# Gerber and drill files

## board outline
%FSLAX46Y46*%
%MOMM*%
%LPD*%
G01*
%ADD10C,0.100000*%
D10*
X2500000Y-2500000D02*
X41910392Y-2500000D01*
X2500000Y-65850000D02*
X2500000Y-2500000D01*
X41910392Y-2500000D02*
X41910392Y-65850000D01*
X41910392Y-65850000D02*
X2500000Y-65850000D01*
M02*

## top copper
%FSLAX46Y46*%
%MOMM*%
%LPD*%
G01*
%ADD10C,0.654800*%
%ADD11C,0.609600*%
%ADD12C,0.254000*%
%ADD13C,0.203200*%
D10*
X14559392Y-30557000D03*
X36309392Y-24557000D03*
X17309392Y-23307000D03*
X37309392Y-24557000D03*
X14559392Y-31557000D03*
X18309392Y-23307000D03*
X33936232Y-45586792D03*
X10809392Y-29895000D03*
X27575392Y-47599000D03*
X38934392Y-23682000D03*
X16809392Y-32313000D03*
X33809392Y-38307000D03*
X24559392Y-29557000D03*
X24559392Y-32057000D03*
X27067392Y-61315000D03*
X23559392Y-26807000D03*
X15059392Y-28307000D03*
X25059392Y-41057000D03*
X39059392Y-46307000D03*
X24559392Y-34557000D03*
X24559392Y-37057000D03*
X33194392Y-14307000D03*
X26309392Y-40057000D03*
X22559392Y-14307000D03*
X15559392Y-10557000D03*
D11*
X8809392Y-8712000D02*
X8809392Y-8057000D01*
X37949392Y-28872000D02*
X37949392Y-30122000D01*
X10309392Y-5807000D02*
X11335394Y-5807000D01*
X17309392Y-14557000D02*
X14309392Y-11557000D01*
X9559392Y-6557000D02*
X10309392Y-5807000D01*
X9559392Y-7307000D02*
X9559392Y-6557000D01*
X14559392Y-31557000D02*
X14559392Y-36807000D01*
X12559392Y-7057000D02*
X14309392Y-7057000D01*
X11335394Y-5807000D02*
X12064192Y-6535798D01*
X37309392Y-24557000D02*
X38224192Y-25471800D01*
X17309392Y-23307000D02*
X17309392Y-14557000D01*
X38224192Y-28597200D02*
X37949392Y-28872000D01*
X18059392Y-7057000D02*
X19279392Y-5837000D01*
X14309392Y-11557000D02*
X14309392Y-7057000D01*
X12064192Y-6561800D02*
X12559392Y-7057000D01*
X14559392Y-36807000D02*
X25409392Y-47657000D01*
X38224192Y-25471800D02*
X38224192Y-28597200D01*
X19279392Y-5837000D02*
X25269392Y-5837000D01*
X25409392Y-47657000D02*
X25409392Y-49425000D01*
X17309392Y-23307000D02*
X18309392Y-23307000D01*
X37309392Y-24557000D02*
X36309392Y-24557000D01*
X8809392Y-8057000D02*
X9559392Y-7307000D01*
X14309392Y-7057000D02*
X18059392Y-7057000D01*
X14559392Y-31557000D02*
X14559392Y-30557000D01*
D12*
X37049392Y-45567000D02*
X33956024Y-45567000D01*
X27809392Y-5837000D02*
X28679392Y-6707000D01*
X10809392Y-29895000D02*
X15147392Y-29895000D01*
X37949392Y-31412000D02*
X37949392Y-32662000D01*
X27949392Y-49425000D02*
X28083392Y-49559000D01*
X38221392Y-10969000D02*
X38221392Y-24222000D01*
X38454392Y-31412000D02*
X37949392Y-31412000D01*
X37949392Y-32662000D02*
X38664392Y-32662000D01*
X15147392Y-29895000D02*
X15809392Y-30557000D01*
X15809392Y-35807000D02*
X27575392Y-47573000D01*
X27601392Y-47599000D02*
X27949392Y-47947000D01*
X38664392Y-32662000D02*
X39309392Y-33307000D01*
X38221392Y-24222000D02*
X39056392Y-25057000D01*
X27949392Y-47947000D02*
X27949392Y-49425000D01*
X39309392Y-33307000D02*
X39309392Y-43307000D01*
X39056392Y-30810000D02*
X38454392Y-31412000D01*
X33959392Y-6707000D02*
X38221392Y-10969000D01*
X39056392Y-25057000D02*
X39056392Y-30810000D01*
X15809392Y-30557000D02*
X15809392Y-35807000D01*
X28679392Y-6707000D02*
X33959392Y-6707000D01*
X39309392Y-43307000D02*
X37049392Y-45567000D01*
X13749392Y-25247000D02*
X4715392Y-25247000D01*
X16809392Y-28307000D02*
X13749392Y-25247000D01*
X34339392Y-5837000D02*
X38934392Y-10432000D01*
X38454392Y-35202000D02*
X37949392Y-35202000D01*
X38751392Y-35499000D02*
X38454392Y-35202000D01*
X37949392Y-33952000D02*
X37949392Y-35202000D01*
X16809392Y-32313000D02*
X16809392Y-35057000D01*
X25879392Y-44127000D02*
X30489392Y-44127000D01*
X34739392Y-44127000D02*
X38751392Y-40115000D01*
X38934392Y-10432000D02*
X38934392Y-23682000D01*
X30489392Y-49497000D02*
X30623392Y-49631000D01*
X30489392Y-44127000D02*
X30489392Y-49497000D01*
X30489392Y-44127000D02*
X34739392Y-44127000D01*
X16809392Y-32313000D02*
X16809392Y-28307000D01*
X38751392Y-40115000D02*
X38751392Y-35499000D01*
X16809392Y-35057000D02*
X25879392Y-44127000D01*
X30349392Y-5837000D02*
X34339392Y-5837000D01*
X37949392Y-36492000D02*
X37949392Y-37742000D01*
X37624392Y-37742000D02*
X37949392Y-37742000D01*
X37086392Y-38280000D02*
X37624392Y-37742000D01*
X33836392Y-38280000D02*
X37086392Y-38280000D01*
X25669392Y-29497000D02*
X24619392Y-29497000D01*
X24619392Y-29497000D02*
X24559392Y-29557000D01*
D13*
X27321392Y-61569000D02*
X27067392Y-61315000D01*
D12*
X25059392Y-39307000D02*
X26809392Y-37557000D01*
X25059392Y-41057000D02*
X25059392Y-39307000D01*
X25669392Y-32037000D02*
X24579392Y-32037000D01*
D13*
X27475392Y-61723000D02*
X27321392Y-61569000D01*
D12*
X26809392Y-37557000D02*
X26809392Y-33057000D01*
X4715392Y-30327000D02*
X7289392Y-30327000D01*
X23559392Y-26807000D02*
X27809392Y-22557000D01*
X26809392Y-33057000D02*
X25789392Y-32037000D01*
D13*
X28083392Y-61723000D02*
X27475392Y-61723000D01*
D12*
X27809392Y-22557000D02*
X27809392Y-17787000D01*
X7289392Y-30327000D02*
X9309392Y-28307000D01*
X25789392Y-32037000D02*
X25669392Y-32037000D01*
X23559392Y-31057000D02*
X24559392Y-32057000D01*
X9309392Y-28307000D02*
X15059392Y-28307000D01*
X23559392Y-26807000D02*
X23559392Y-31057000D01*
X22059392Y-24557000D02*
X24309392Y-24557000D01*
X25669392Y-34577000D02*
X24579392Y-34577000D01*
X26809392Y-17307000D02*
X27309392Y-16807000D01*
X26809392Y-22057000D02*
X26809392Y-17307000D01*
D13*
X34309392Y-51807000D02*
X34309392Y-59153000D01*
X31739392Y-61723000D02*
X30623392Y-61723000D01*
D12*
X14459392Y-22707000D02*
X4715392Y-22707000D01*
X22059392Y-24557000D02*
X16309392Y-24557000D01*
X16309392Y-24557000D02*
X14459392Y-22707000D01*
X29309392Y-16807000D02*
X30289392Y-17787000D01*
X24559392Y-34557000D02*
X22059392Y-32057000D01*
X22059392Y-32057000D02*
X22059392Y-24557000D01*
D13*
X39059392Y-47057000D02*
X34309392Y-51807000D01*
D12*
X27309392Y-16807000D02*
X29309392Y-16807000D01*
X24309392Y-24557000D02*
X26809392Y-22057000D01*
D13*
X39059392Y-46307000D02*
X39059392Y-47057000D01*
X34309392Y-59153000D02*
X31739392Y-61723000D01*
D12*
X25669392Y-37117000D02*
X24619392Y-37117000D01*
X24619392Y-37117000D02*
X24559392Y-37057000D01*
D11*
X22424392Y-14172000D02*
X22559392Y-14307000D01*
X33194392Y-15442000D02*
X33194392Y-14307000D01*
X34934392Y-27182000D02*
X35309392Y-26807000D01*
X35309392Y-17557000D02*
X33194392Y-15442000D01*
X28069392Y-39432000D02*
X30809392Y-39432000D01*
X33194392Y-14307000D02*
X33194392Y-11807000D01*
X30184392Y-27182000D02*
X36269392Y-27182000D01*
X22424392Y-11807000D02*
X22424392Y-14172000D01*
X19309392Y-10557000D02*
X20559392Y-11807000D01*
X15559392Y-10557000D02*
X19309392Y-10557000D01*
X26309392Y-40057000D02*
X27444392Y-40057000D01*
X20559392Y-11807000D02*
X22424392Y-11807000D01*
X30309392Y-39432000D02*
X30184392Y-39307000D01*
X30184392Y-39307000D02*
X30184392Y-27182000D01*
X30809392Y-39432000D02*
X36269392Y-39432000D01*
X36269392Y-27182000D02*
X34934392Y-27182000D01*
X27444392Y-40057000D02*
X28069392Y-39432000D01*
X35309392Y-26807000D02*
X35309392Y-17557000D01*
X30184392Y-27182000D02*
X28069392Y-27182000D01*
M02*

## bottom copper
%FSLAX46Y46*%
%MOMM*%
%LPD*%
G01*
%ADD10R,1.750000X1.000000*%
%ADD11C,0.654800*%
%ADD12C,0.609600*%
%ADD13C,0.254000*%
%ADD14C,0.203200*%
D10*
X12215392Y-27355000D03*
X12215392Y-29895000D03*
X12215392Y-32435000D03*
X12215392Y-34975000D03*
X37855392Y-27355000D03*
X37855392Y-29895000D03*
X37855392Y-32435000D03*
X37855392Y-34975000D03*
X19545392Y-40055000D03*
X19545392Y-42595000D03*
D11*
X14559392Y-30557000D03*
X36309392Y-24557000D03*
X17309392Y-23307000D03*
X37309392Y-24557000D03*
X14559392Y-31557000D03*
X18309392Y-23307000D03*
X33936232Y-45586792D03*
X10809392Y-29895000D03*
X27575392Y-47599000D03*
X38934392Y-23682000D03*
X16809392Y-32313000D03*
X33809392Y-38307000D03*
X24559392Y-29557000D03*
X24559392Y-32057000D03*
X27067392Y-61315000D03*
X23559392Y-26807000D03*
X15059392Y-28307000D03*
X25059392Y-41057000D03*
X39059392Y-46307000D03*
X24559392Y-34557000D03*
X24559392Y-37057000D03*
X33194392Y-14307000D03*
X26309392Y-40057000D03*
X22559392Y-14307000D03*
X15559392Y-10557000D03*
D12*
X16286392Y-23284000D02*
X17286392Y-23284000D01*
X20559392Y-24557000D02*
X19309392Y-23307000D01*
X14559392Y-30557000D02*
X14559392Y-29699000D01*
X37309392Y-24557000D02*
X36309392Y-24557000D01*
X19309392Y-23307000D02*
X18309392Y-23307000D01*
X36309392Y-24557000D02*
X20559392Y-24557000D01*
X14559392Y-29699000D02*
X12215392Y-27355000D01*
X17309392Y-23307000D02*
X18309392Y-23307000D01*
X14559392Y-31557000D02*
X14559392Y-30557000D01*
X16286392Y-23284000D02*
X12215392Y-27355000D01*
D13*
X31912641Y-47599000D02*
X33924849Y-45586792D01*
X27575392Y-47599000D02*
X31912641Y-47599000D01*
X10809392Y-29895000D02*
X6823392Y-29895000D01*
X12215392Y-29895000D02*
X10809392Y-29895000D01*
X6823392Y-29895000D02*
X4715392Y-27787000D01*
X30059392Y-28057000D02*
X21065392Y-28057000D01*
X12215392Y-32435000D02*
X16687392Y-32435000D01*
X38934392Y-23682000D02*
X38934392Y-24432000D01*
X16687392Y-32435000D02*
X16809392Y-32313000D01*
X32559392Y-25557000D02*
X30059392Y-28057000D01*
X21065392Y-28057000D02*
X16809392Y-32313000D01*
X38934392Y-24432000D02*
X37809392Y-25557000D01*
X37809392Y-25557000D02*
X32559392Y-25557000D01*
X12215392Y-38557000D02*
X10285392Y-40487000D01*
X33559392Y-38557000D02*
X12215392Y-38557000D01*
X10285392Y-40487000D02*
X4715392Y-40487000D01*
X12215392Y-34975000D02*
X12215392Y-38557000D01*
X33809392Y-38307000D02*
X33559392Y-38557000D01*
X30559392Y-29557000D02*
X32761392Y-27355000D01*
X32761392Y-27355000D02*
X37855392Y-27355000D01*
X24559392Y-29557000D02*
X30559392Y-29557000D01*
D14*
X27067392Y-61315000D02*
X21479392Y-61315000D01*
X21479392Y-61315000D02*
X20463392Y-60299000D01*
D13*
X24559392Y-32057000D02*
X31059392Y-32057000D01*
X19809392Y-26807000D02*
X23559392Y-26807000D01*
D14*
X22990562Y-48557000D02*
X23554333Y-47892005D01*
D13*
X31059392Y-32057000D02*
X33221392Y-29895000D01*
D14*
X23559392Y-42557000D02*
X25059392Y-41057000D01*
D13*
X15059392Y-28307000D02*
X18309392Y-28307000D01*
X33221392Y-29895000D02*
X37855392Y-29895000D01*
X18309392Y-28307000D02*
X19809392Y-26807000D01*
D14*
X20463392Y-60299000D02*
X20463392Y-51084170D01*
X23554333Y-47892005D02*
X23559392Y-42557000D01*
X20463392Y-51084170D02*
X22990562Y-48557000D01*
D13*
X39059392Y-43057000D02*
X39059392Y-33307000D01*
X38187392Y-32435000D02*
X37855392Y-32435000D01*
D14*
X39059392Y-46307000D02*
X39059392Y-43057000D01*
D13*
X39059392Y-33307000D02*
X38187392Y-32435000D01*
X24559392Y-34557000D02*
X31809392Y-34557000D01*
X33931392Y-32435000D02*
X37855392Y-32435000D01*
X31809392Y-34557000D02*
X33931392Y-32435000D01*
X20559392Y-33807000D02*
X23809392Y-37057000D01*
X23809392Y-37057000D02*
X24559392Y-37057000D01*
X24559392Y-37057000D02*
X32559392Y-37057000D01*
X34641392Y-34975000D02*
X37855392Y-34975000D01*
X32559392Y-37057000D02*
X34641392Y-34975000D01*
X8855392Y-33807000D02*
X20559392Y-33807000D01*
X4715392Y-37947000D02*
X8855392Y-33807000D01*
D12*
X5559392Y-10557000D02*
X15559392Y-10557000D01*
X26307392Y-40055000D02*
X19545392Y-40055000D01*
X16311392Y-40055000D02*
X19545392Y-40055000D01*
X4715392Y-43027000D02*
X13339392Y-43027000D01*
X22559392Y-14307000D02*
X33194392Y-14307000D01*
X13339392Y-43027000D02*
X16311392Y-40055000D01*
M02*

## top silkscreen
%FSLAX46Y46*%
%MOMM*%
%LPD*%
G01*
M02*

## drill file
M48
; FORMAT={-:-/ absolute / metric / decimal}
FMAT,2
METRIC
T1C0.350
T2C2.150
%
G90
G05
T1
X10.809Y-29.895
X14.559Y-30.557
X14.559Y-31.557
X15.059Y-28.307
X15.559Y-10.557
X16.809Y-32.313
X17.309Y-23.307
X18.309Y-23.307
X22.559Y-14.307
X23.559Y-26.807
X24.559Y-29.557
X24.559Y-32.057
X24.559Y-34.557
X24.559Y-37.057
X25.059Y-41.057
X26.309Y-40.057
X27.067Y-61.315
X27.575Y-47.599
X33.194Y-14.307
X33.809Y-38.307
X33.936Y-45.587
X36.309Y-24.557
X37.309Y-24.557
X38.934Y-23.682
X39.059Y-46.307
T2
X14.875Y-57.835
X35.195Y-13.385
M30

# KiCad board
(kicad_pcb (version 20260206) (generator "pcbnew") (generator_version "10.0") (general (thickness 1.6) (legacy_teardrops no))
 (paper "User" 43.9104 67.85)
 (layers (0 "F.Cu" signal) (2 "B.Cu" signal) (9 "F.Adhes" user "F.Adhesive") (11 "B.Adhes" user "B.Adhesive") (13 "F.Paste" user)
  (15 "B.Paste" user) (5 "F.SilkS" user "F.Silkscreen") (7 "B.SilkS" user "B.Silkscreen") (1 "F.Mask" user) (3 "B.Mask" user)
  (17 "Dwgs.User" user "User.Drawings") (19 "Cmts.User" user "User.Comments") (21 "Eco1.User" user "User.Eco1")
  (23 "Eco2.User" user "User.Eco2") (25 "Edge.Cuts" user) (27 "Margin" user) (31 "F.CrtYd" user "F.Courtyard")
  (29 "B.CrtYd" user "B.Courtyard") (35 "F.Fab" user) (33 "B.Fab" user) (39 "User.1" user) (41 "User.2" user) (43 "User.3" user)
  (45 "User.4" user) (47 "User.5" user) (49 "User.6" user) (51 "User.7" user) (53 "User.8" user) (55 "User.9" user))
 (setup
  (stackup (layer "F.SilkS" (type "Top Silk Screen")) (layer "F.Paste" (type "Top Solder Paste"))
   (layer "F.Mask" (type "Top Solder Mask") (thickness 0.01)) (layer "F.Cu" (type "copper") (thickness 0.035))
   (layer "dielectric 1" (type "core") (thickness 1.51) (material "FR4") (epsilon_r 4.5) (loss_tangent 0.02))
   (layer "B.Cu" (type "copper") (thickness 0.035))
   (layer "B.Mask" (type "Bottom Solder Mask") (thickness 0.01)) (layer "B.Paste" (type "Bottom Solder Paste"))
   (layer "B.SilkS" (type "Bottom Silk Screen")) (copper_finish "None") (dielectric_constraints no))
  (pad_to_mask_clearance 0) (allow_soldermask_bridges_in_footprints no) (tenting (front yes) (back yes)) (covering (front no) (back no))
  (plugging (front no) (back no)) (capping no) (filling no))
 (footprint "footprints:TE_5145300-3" (layer "B.Cu") (at 23.085392 34.175 -90)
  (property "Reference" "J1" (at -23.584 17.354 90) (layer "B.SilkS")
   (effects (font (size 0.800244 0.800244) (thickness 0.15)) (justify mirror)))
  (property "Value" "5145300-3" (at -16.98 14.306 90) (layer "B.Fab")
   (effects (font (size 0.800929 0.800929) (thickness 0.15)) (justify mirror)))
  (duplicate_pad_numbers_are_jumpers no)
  (pad "" np_thru_hole circle (at -20.79 -12.11 270) (size 2.15 2.15) (drill 2.15) (layers "*.Cu" "*.Mask"))
  (pad "" np_thru_hole circle (at 23.66 8.21 270) (size 2.15 2.15) (drill 2.15) (layers "*.Cu" "*.Mask"))
  (pad "C1" smd rect (at -6.82 10.87 180) (size 1.75 1) (layers "B.Cu" "B.Mask" "B.Paste") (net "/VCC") (solder_mask_margin 0.102))
  (pad "C2" smd rect (at -4.28 10.87 180) (size 1.75 1) (layers "B.Cu" "B.Mask" "B.Paste") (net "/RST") (solder_mask_margin 0.102))
  (pad "C3" smd rect (at -1.74 10.87 180) (size 1.75 1) (layers "B.Cu" "B.Mask" "B.Paste") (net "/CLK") (solder_mask_margin 0.102))
  (pad "C4" smd rect (at 0.8 10.87 180) (size 1.75 1) (layers "B.Cu" "B.Mask" "B.Paste") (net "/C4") (solder_mask_margin 0.102))
  (pad "C5" smd rect (at -6.82 -14.77 180) (size 1.75 1) (layers "B.Cu" "B.Mask" "B.Paste") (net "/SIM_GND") (solder_mask_margin 0.102))
  (pad "C6" smd rect (at -4.28 -14.77 180) (size 1.75 1) (layers "B.Cu" "B.Mask" "B.Paste") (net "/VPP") (solder_mask_margin 0.102))
  (pad "C7" smd rect (at -1.74 -14.77 180) (size 1.75 1) (layers "B.Cu" "B.Mask" "B.Paste") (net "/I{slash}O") (solder_mask_margin 0.102))
  (pad "C8" smd rect (at 0.8 -14.77 180) (size 1.75 1) (layers "B.Cu" "B.Mask" "B.Paste") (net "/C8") (solder_mask_margin 0.102))
  (pad "SW1" smd rect (at 5.88 3.54 180) (size 1.75 1) (layers "B.Cu" "B.Mask" "B.Paste") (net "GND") (solder_mask_margin 0.102))
  (pad "SW2" smd rect (at 8.42 3.54 180) (size 1.75 1) (layers "B.Cu" "B.Mask" "B.Paste") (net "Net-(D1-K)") (solder_mask_margin 0.102)))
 (gr_line (start 2.5 2.5) (end 41.910392 2.5) (stroke (width 0.1) (type default)) (layer "Edge.Cuts"))
 (gr_line (start 2.5 65.85) (end 2.5 2.5) (stroke (width 0.1) (type default)) (layer "Edge.Cuts"))
 (gr_line (start 41.910392 2.5) (end 41.910392 65.85) (stroke (width 0.1) (type default)) (layer "Edge.Cuts"))
 (gr_line (start 41.910392 65.85) (end 2.5 65.85) (stroke (width 0.1) (type default)) (layer "Edge.Cuts"))
 (segment (start 8.809392 8.712) (end 8.809392 8.057) (width 0.6096) (layer "F.Cu") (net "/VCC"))
 (segment (start 37.949392 28.872) (end 37.949392 30.122) (width 0.6096) (layer "F.Cu") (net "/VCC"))
 (segment (start 10.309392 5.807) (end 11.335394 5.807) (width 0.6096) (layer "F.Cu") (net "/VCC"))
 (segment (start 17.309392 14.557) (end 14.309392 11.557) (width 0.6096) (layer "F.Cu") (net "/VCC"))
 (segment (start 9.559392 6.557) (end 10.309392 5.807) (width 0.6096) (layer "F.Cu") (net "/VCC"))
 (segment (start 9.559392 7.307) (end 9.559392 6.557) (width 0.6096) (layer "F.Cu") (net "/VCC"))
 (segment (start 14.559392 31.557) (end 14.559392 36.807) (width 0.6096) (layer "F.Cu") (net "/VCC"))
 (segment (start 12.559392 7.057) (end 14.309392 7.057) (width 0.6096) (layer "F.Cu") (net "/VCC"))
 (segment (start 11.335394 5.807) (end 12.064192 6.535798) (width 0.6096) (layer "F.Cu") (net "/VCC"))
 (segment (start 37.309392 24.557) (end 38.224192 25.4718) (width 0.6096) (layer "F.Cu") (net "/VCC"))
 (segment (start 17.309392 23.307) (end 17.309392 14.557) (width 0.6096) (layer "F.Cu") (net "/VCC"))
 (segment (start 38.224192 28.5972) (end 37.949392 28.872) (width 0.6096) (layer "F.Cu") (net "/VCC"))
 (segment (start 18.059392 7.057) (end 19.279392 5.837) (width 0.6096) (layer "F.Cu") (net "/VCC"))
 (segment (start 14.309392 11.557) (end 14.309392 7.057) (width 0.6096) (layer "F.Cu") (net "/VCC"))
 (segment (start 12.064192 6.5618) (end 12.559392 7.057) (width 0.6096) (layer "F.Cu") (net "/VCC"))
 (segment (start 14.559392 36.807) (end 25.409392 47.657) (width 0.6096) (layer "F.Cu") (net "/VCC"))
 (segment (start 38.224192 25.4718) (end 38.224192 28.5972) (width 0.6096) (layer "F.Cu") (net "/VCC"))
 (segment (start 19.279392 5.837) (end 25.269392 5.837) (width 0.6096) (layer "F.Cu") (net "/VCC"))
 (segment (start 25.409392 47.657) (end 25.409392 49.425) (width 0.6096) (layer "F.Cu") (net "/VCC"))
 (segment (start 17.309392 23.307) (end 18.309392 23.307) (width 0.6096) (layer "F.Cu") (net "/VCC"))
 (segment (start 37.309392 24.557) (end 36.309392 24.557) (width 0.6096) (layer "F.Cu") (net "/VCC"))
 (segment (start 8.809392 8.057) (end 9.559392 7.307) (width 0.6096) (layer "F.Cu") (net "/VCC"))
 (segment (start 14.309392 7.057) (end 18.059392 7.057) (width 0.6096) (layer "F.Cu") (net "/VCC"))
 (segment (start 14.559392 31.557) (end 14.559392 30.557) (width 0.6096) (layer "F.Cu") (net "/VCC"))
 (via (at 14.559392 30.557) (size 0.6548) (drill 0.35) (layers "F.Cu" "B.Cu") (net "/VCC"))
 (via (at 36.309392 24.557) (size 0.6548) (drill 0.35) (layers "F.Cu" "B.Cu") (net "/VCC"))
 (via (at 17.309392 23.307) (size 0.6548) (drill 0.35) (layers "F.Cu" "B.Cu") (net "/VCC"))
 (via (at 37.309392 24.557) (size 0.6548) (drill 0.35) (layers "F.Cu" "B.Cu") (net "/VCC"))
 (via (at 14.559392 31.557) (size 0.6548) (drill 0.35) (layers "F.Cu" "B.Cu") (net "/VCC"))
 (via (at 18.309392 23.307) (size 0.6548) (drill 0.35) (layers "F.Cu" "B.Cu") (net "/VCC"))
 (segment (start 16.286392 23.284) (end 17.286392 23.284) (width 0.6096) (layer "B.Cu") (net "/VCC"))
 (segment (start 20.559392 24.557) (end 19.309392 23.307) (width 0.6096) (layer "B.Cu") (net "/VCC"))
 (segment (start 14.559392 30.557) (end 14.559392 29.699) (width 0.6096) (layer "B.Cu") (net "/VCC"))
 (segment (start 37.309392 24.557) (end 36.309392 24.557) (width 0.6096) (layer "B.Cu") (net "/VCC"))
 (segment (start 19.309392 23.307) (end 18.309392 23.307) (width 0.6096) (layer "B.Cu") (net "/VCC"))
 (segment (start 36.309392 24.557) (end 20.559392 24.557) (width 0.6096) (layer "B.Cu") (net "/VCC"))
 (segment (start 14.559392 29.699) (end 12.215392 27.355) (width 0.6096) (layer "B.Cu") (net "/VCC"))
 (segment (start 17.309392 23.307) (end 18.309392 23.307) (width 0.6096) (layer "B.Cu") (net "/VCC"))
 (segment (start 14.559392 31.557) (end 14.559392 30.557) (width 0.6096) (layer "B.Cu") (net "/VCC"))
 (segment (start 16.286392 23.284) (end 12.215392 27.355) (width 0.6096) (layer "B.Cu") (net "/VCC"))
 (segment (start 37.049392 45.567) (end 33.956024 45.567) (width 0.254) (layer "F.Cu") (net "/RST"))
 (segment (start 27.809392 5.837) (end 28.679392 6.707) (width 0.254) (layer "F.Cu") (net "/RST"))
 (segment (start 10.809392 29.895) (end 15.147392 29.895) (width 0.254) (layer "F.Cu") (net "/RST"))
 (segment (start 37.949392 31.412) (end 37.949392 32.662) (width 0.254) (layer "F.Cu") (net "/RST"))
 (segment (start 27.949392 49.425) (end 28.083392 49.559) (width 0.254) (layer "F.Cu") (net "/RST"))
 (segment (start 38.221392 10.969) (end 38.221392 24.222) (width 0.254) (layer "F.Cu") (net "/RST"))
 (segment (start 38.454392 31.412) (end 37.949392 31.412) (width 0.254) (layer "F.Cu") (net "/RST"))
 (segment (start 37.949392 32.662) (end 38.664392 32.662) (width 0.254) (layer "F.Cu") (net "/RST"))
 (segment (start 15.147392 29.895) (end 15.809392 30.557) (width 0.254) (layer "F.Cu") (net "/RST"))
 (segment (start 15.809392 35.807) (end 27.575392 47.573) (width 0.254) (layer "F.Cu") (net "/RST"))
 (segment (start 27.601392 47.599) (end 27.949392 47.947) (width 0.254) (layer "F.Cu") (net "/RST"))
 (segment (start 38.664392 32.662) (end 39.309392 33.307) (width 0.254) (layer "F.Cu") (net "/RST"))
 (segment (start 38.221392 24.222) (end 39.056392 25.057) (width 0.254) (layer "F.Cu") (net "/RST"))
 (segment (start 27.949392 47.947) (end 27.949392 49.425) (width 0.254) (layer "F.Cu") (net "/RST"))
 (segment (start 39.309392 33.307) (end 39.309392 43.307) (width 0.254) (layer "F.Cu") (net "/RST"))
 (segment (start 39.056392 30.81) (end 38.454392 31.412) (width 0.254) (layer "F.Cu") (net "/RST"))
 (segment (start 33.959392 6.707) (end 38.221392 10.969) (width 0.254) (layer "F.Cu") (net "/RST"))
 (segment (start 39.056392 25.057) (end 39.056392 30.81) (width 0.254) (layer "F.Cu") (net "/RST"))
 (segment (start 15.809392 30.557) (end 15.809392 35.807) (width 0.254) (layer "F.Cu") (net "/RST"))
 (segment (start 28.679392 6.707) (end 33.959392 6.707) (width 0.254) (layer "F.Cu") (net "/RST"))
 (segment (start 39.309392 43.307) (end 37.049392 45.567) (width 0.254) (layer "F.Cu") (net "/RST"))
 (via (at 33.936232 45.586792) (size 0.6548) (drill 0.35) (layers "F.Cu" "B.Cu") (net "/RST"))
 (via (at 10.809392 29.895) (size 0.6548) (drill 0.35) (layers "F.Cu" "B.Cu") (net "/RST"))
 (via (at 27.575392 47.599) (size 0.6548) (drill 0.35) (layers "F.Cu" "B.Cu") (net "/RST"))
 (segment (start 31.912641 47.599) (end 33.924849 45.586792) (width 0.254) (layer "B.Cu") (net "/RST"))
 (segment (start 27.575392 47.599) (end 31.912641 47.599) (width 0.254) (layer "B.Cu") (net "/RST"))
 (segment (start 10.809392 29.895) (end 6.823392 29.895) (width 0.254) (layer "B.Cu") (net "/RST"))
 (segment (start 12.215392 29.895) (end 10.809392 29.895) (width 0.254) (layer "B.Cu") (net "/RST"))
 (segment (start 6.823392 29.895) (end 4.715392 27.787) (width 0.254) (layer "B.Cu") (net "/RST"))
 (segment (start 13.749392 25.247) (end 4.715392 25.247) (width 0.254) (layer "F.Cu") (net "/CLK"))
 (segment (start 16.809392 28.307) (end 13.749392 25.247) (width 0.254) (layer "F.Cu") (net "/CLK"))
 (segment (start 34.339392 5.837) (end 38.934392 10.432) (width 0.254) (layer "F.Cu") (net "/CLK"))
 (segment (start 38.454392 35.202) (end 37.949392 35.202) (width 0.254) (layer "F.Cu") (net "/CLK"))
 (segment (start 38.751392 35.499) (end 38.454392 35.202) (width 0.254) (layer "F.Cu") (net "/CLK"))
 (segment (start 37.949392 33.952) (end 37.949392 35.202) (width 0.254) (layer "F.Cu") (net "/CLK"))
 (segment (start 16.809392 32.313) (end 16.809392 35.057) (width 0.254) (layer "F.Cu") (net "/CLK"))
 (segment (start 25.879392 44.127) (end 30.489392 44.127) (width 0.254) (layer "F.Cu") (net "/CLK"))
 (segment (start 34.739392 44.127) (end 38.751392 40.115) (width 0.254) (layer "F.Cu") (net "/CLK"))
 (segment (start 38.934392 10.432) (end 38.934392 23.682) (width 0.254) (layer "F.Cu") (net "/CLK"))
 (segment (start 30.489392 49.497) (end 30.623392 49.631) (width 0.254) (layer "F.Cu") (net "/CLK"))
 (segment (start 30.489392 44.127) (end 30.489392 49.497) (width 0.254) (layer "F.Cu") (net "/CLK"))
 (segment (start 30.489392 44.127) (end 34.739392 44.127) (width 0.254) (layer "F.Cu") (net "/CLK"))
 (segment (start 16.809392 32.313) (end 16.809392 28.307) (width 0.254) (layer "F.Cu") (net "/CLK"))
 (segment (start 38.751392 40.115) (end 38.751392 35.499) (width 0.254) (layer "F.Cu") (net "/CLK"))
 (segment (start 16.809392 35.057) (end 25.879392 44.127) (width 0.254) (layer "F.Cu") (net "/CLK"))
 (segment (start 30.349392 5.837) (end 34.339392 5.837) (width 0.254) (layer "F.Cu") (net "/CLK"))
 (via (at 38.934392 23.682) (size 0.6548) (drill 0.35) (layers "F.Cu" "B.Cu") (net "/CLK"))
 (via (at 16.809392 32.313) (size 0.6548) (drill 0.35) (layers "F.Cu" "B.Cu") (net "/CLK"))
 (segment (start 30.059392 28.057) (end 21.065392 28.057) (width 0.254) (layer "B.Cu") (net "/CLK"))
 (segment (start 12.215392 32.435) (end 16.687392 32.435) (width 0.254) (layer "B.Cu") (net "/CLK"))
 (segment (start 38.934392 23.682) (end 38.934392 24.432) (width 0.254) (layer "B.Cu") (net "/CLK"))
 (segment (start 16.687392 32.435) (end 16.809392 32.313) (width 0.254) (layer "B.Cu") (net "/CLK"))
 (segment (start 32.559392 25.557) (end 30.059392 28.057) (width 0.254) (layer "B.Cu") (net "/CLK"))
 (segment (start 21.065392 28.057) (end 16.809392 32.313) (width 0.254) (layer "B.Cu") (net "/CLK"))
 (segment (start 38.934392 24.432) (end 37.809392 25.557) (width 0.254) (layer "B.Cu") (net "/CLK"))
 (segment (start 37.809392 25.557) (end 32.559392 25.557) (width 0.254) (layer "B.Cu") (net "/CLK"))
 (segment (start 37.949392 36.492) (end 37.949392 37.742) (width 0.254) (layer "F.Cu") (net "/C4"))
 (segment (start 37.624392 37.742) (end 37.949392 37.742) (width 0.254) (layer "F.Cu") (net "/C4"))
 (segment (start 37.086392 38.28) (end 37.624392 37.742) (width 0.254) (layer "F.Cu") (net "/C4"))
 (segment (start 33.836392 38.28) (end 37.086392 38.28) (width 0.254) (layer "F.Cu") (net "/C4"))
 (via (at 33.809392 38.307) (size 0.6548) (drill 0.35) (layers "F.Cu" "B.Cu") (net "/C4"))
 (segment (start 12.215392 38.557) (end 10.285392 40.487) (width 0.254) (layer "B.Cu") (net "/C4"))
 (segment (start 33.559392 38.557) (end 12.215392 38.557) (width 0.254) (layer "B.Cu") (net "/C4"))
 (segment (start 10.285392 40.487) (end 4.715392 40.487) (width 0.254) (layer "B.Cu") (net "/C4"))
 (segment (start 12.215392 34.975) (end 12.215392 38.557) (width 0.254) (layer "B.Cu") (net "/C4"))
 (segment (start 33.809392 38.307) (end 33.559392 38.557) (width 0.254) (layer "B.Cu") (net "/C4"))
 (segment (start 25.669392 29.497) (end 24.619392 29.497) (width 0.254) (layer "F.Cu") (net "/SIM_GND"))
 (segment (start 24.619392 29.497) (end 24.559392 29.557) (width 0.254) (layer "F.Cu") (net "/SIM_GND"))
 (via (at 24.559392 29.557) (size 0.6548) (drill 0.35) (layers "F.Cu" "B.Cu") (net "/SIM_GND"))
 (segment (start 30.559392 29.557) (end 32.761392 27.355) (width 0.254) (layer "B.Cu") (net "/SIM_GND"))
 (segment (start 32.761392 27.355) (end 37.855392 27.355) (width 0.254) (layer "B.Cu") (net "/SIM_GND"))
 (segment (start 24.559392 29.557) (end 30.559392 29.557) (width 0.254) (layer "B.Cu") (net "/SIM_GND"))
 (segment (start 27.321392 61.569) (end 27.067392 61.315) (width 0.2032) (layer "F.Cu") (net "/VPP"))
 (segment (start 25.059392 39.307) (end 26.809392 37.557) (width 0.254) (layer "F.Cu") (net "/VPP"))
 (segment (start 25.059392 41.057) (end 25.059392 39.307) (width 0.254) (layer "F.Cu") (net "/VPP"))
 (segment (start 25.669392 32.037) (end 24.579392 32.037) (width 0.254) (layer "F.Cu") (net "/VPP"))
 (segment (start 27.475392 61.723) (end 27.321392 61.569) (width 0.2032) (layer "F.Cu") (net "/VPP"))
 (segment (start 26.809392 37.557) (end 26.809392 33.057) (width 0.254) (layer "F.Cu") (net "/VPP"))
 (segment (start 4.715392 30.327) (end 7.289392 30.327) (width 0.254) (layer "F.Cu") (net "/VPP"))
 (segment (start 23.559392 26.807) (end 27.809392 22.557) (width 0.254) (layer "F.Cu") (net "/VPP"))
 (segment (start 26.809392 33.057) (end 25.789392 32.037) (width 0.254) (layer "F.Cu") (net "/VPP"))
 (segment (start 28.083392 61.723) (end 27.475392 61.723) (width 0.2032) (layer "F.Cu") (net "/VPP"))
 (segment (start 27.809392 22.557) (end 27.809392 17.787) (width 0.254) (layer "F.Cu") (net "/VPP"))
 (segment (start 7.289392 30.327) (end 9.309392 28.307) (width 0.254) (layer "F.Cu") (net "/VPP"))
 (segment (start 25.789392 32.037) (end 25.669392 32.037) (width 0.254) (layer "F.Cu") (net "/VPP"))
 (segment (start 23.559392 31.057) (end 24.559392 32.057) (width 0.254) (layer "F.Cu") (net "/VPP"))
 (segment (start 9.309392 28.307) (end 15.059392 28.307) (width 0.254) (layer "F.Cu") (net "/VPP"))
 (segment (start 23.559392 26.807) (end 23.559392 31.057) (width 0.254) (layer "F.Cu") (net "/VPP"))
 (via (at 24.559392 32.057) (size 0.6548) (drill 0.35) (layers "F.Cu" "B.Cu") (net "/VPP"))
 (via (at 27.067392 61.315) (size 0.6548) (drill 0.35) (layers "F.Cu" "B.Cu") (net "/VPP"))
 (via (at 23.559392 26.807) (size 0.6548) (drill 0.35) (layers "F.Cu" "B.Cu") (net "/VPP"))
 (via (at 15.059392 28.307) (size 0.6548) (drill 0.35) (layers "F.Cu" "B.Cu") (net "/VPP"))
 (via (at 25.059392 41.057) (size 0.6548) (drill 0.35) (layers "F.Cu" "B.Cu") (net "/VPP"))
 (segment (start 27.067392 61.315) (end 21.479392 61.315) (width 0.2032) (layer "B.Cu") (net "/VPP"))
 (segment (start 21.479392 61.315) (end 20.463392 60.299) (width 0.2032) (layer "B.Cu") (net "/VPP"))
 (segment (start 24.559392 32.057) (end 31.059392 32.057) (width 0.254) (layer "B.Cu") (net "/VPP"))
 (segment (start 19.809392 26.807) (end 23.559392 26.807) (width 0.254) (layer "B.Cu") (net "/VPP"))
 (segment (start 22.990562 48.557) (end 23.554333 47.892005) (width 0.2032) (layer "B.Cu") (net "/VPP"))
 (segment (start 31.059392 32.057) (end 33.221392 29.895) (width 0.254) (layer "B.Cu") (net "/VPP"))
 (segment (start 23.559392 42.557) (end 25.059392 41.057) (width 0.2032) (layer "B.Cu") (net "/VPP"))
 (segment (start 15.059392 28.307) (end 18.309392 28.307) (width 0.254) (layer "B.Cu") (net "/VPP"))
 (segment (start 33.221392 29.895) (end 37.855392 29.895) (width 0.254) (layer "B.Cu") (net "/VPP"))
 (segment (start 18.309392 28.307) (end 19.809392 26.807) (width 0.254) (layer "B.Cu") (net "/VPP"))
 (segment (start 20.463392 60.299) (end 20.463392 51.08417) (width 0.2032) (layer "B.Cu") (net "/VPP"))
 (segment (start 23.554333 47.892005) (end 23.559392 42.557) (width 0.2032) (layer "B.Cu") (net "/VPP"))
 (segment (start 20.463392 51.08417) (end 22.990562 48.557) (width 0.2032) (layer "B.Cu") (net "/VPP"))
 (segment (start 22.059392 24.557) (end 24.309392 24.557) (width 0.254) (layer "F.Cu") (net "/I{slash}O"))
 (segment (start 25.669392 34.577) (end 24.579392 34.577) (width 0.254) (layer "F.Cu") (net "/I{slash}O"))
 (segment (start 26.809392 17.307) (end 27.309392 16.807) (width 0.254) (layer "F.Cu") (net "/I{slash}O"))
 (segment (start 26.809392 22.057) (end 26.809392 17.307) (width 0.254) (layer "F.Cu") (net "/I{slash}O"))
 (segment (start 34.309392 51.807) (end 34.309392 59.153) (width 0.2032) (layer "F.Cu") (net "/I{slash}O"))
 (segment (start 31.739392 61.723) (end 30.623392 61.723) (width 0.2032) (layer "F.Cu") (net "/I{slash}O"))
 (segment (start 14.459392 22.707) (end 4.715392 22.707) (width 0.254) (layer "F.Cu") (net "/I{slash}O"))
 (segment (start 22.059392 24.557) (end 16.309392 24.557) (width 0.254) (layer "F.Cu") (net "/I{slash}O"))
 (segment (start 16.309392 24.557) (end 14.459392 22.707) (width 0.254) (layer "F.Cu") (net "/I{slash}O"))
 (segment (start 29.309392 16.807) (end 30.289392 17.787) (width 0.254) (layer "F.Cu") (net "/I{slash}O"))
 (segment (start 24.559392 34.557) (end 22.059392 32.057) (width 0.254) (layer "F.Cu") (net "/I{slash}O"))
 (segment (start 22.059392 32.057) (end 22.059392 24.557) (width 0.254) (layer "F.Cu") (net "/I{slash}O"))
 (segment (start 39.059392 47.057) (end 34.309392 51.807) (width 0.2032) (layer "F.Cu") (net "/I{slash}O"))
 (segment (start 27.309392 16.807) (end 29.309392 16.807) (width 0.254) (layer "F.Cu") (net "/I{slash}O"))
 (segment (start 24.309392 24.557) (end 26.809392 22.057) (width 0.254) (layer "F.Cu") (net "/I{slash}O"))
 (segment (start 39.059392 46.307) (end 39.059392 47.057) (width 0.2032) (layer "F.Cu") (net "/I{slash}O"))
 (segment (start 34.309392 59.153) (end 31.739392 61.723) (width 0.2032) (layer "F.Cu") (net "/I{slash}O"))
 (via (at 39.059392 46.307) (size 0.6548) (drill 0.35) (layers "F.Cu" "B.Cu") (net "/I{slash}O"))
 (via (at 24.559392 34.557) (size 0.6548) (drill 0.35) (layers "F.Cu" "B.Cu") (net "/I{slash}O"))
 (segment (start 39.059392 43.057) (end 39.059392 33.307) (width 0.254) (layer "B.Cu") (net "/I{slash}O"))
 (segment (start 38.187392 32.435) (end 37.855392 32.435) (width 0.254) (layer "B.Cu") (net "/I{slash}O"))
 (segment (start 39.059392 46.307) (end 39.059392 43.057) (width 0.2032) (layer "B.Cu") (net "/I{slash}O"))
 (segment (start 39.059392 33.307) (end 38.187392 32.435) (width 0.254) (layer "B.Cu") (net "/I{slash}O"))
 (segment (start 24.559392 34.557) (end 31.809392 34.557) (width 0.254) (layer "B.Cu") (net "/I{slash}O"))
 (segment (start 33.931392 32.435) (end 37.855392 32.435) (width 0.254) (layer "B.Cu") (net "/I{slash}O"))
 (segment (start 31.809392 34.557) (end 33.931392 32.435) (width 0.254) (layer "B.Cu") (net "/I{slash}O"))
 (segment (start 25.669392 37.117) (end 24.619392 37.117) (width 0.254) (layer "F.Cu") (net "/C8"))
 (segment (start 24.619392 37.117) (end 24.559392 37.057) (width 0.254) (layer "F.Cu") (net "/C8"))
 (via (at 24.559392 37.057) (size 0.6548) (drill 0.35) (layers "F.Cu" "B.Cu") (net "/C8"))
 (segment (start 20.559392 33.807) (end 23.809392 37.057) (width 0.254) (layer "B.Cu") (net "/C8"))
 (segment (start 23.809392 37.057) (end 24.559392 37.057) (width 0.254) (layer "B.Cu") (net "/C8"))
 (segment (start 24.559392 37.057) (end 32.559392 37.057) (width 0.254) (layer "B.Cu") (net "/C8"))
 (segment (start 34.641392 34.975) (end 37.855392 34.975) (width 0.254) (layer "B.Cu") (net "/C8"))
 (segment (start 32.559392 37.057) (end 34.641392 34.975) (width 0.254) (layer "B.Cu") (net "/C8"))
 (segment (start 8.855392 33.807) (end 20.559392 33.807) (width 0.254) (layer "B.Cu") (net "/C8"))
 (segment (start 4.715392 37.947) (end 8.855392 33.807) (width 0.254) (layer "B.Cu") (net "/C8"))
 (segment (start 22.424392 14.172) (end 22.559392 14.307) (width 0.6096) (layer "F.Cu") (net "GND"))
 (segment (start 33.194392 15.442) (end 33.194392 14.307) (width 0.6096) (layer "F.Cu") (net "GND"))
 (segment (start 34.934392 27.182) (end 35.309392 26.807) (width 0.6096) (layer "F.Cu") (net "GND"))
 (segment (start 35.309392 17.557) (end 33.194392 15.442) (width 0.6096) (layer "F.Cu") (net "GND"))
 (segment (start 28.069392 39.432) (end 30.809392 39.432) (width 0.6096) (layer "F.Cu") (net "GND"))
 (segment (start 33.194392 14.307) (end 33.194392 11.807) (width 0.6096) (layer "F.Cu") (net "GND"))
 (segment (start 30.184392 27.182) (end 36.269392 27.182) (width 0.6096) (layer "F.Cu") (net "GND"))
 (segment (start 22.424392 11.807) (end 22.424392 14.172) (width 0.6096) (layer "F.Cu") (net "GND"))
 (segment (start 19.309392 10.557) (end 20.559392 11.807) (width 0.6096) (layer "F.Cu") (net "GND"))
 (segment (start 15.559392 10.557) (end 19.309392 10.557) (width 0.6096) (layer "F.Cu") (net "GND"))
 (segment (start 26.309392 40.057) (end 27.444392 40.057) (width 0.6096) (layer "F.Cu") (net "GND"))
 (segment (start 20.559392 11.807) (end 22.424392 11.807) (width 0.6096) (layer "F.Cu") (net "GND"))
 (segment (start 30.309392 39.432) (end 30.184392 39.307) (width 0.6096) (layer "F.Cu") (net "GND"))
 (segment (start 30.184392 39.307) (end 30.184392 27.182) (width 0.6096) (layer "F.Cu") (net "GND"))
 (segment (start 30.809392 39.432) (end 36.269392 39.432) (width 0.6096) (layer "F.Cu") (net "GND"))
 (segment (start 36.269392 27.182) (end 34.934392 27.182) (width 0.6096) (layer "F.Cu") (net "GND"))
 (segment (start 27.444392 40.057) (end 28.069392 39.432) (width 0.6096) (layer "F.Cu") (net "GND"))
 (segment (start 35.309392 26.807) (end 35.309392 17.557) (width 0.6096) (layer "F.Cu") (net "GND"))
 (segment (start 30.184392 27.182) (end 28.069392 27.182) (width 0.6096) (layer "F.Cu") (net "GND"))
 (via (at 33.194392 14.307) (size 0.6548) (drill 0.35) (layers "F.Cu" "B.Cu") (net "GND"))
 (via (at 26.309392 40.057) (size 0.6548) (drill 0.35) (layers "F.Cu" "B.Cu") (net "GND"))
 (via (at 22.559392 14.307) (size 0.6548) (drill 0.35) (layers "F.Cu" "B.Cu") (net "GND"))
 (via (at 15.559392 10.557) (size 0.6548) (drill 0.35) (layers "F.Cu" "B.Cu") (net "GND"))
 (segment (start 5.559392 10.557) (end 15.559392 10.557) (width 0.6096) (layer "B.Cu") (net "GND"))
 (segment (start 26.307392 40.055) (end 19.545392 40.055) (width 0.6096) (layer "B.Cu") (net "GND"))
 (segment (start 16.311392 40.055) (end 19.545392 40.055) (width 0.6096) (layer "B.Cu") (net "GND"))
 (segment (start 4.715392 43.027) (end 13.339392 43.027) (width 0.6096) (layer "B.Cu") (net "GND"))
 (segment (start 22.559392 14.307) (end 33.194392 14.307) (width 0.6096) (layer "B.Cu") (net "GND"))
 (segment (start 13.339392 43.027) (end 16.311392 40.055) (width 0.6096) (layer "B.Cu") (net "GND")))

